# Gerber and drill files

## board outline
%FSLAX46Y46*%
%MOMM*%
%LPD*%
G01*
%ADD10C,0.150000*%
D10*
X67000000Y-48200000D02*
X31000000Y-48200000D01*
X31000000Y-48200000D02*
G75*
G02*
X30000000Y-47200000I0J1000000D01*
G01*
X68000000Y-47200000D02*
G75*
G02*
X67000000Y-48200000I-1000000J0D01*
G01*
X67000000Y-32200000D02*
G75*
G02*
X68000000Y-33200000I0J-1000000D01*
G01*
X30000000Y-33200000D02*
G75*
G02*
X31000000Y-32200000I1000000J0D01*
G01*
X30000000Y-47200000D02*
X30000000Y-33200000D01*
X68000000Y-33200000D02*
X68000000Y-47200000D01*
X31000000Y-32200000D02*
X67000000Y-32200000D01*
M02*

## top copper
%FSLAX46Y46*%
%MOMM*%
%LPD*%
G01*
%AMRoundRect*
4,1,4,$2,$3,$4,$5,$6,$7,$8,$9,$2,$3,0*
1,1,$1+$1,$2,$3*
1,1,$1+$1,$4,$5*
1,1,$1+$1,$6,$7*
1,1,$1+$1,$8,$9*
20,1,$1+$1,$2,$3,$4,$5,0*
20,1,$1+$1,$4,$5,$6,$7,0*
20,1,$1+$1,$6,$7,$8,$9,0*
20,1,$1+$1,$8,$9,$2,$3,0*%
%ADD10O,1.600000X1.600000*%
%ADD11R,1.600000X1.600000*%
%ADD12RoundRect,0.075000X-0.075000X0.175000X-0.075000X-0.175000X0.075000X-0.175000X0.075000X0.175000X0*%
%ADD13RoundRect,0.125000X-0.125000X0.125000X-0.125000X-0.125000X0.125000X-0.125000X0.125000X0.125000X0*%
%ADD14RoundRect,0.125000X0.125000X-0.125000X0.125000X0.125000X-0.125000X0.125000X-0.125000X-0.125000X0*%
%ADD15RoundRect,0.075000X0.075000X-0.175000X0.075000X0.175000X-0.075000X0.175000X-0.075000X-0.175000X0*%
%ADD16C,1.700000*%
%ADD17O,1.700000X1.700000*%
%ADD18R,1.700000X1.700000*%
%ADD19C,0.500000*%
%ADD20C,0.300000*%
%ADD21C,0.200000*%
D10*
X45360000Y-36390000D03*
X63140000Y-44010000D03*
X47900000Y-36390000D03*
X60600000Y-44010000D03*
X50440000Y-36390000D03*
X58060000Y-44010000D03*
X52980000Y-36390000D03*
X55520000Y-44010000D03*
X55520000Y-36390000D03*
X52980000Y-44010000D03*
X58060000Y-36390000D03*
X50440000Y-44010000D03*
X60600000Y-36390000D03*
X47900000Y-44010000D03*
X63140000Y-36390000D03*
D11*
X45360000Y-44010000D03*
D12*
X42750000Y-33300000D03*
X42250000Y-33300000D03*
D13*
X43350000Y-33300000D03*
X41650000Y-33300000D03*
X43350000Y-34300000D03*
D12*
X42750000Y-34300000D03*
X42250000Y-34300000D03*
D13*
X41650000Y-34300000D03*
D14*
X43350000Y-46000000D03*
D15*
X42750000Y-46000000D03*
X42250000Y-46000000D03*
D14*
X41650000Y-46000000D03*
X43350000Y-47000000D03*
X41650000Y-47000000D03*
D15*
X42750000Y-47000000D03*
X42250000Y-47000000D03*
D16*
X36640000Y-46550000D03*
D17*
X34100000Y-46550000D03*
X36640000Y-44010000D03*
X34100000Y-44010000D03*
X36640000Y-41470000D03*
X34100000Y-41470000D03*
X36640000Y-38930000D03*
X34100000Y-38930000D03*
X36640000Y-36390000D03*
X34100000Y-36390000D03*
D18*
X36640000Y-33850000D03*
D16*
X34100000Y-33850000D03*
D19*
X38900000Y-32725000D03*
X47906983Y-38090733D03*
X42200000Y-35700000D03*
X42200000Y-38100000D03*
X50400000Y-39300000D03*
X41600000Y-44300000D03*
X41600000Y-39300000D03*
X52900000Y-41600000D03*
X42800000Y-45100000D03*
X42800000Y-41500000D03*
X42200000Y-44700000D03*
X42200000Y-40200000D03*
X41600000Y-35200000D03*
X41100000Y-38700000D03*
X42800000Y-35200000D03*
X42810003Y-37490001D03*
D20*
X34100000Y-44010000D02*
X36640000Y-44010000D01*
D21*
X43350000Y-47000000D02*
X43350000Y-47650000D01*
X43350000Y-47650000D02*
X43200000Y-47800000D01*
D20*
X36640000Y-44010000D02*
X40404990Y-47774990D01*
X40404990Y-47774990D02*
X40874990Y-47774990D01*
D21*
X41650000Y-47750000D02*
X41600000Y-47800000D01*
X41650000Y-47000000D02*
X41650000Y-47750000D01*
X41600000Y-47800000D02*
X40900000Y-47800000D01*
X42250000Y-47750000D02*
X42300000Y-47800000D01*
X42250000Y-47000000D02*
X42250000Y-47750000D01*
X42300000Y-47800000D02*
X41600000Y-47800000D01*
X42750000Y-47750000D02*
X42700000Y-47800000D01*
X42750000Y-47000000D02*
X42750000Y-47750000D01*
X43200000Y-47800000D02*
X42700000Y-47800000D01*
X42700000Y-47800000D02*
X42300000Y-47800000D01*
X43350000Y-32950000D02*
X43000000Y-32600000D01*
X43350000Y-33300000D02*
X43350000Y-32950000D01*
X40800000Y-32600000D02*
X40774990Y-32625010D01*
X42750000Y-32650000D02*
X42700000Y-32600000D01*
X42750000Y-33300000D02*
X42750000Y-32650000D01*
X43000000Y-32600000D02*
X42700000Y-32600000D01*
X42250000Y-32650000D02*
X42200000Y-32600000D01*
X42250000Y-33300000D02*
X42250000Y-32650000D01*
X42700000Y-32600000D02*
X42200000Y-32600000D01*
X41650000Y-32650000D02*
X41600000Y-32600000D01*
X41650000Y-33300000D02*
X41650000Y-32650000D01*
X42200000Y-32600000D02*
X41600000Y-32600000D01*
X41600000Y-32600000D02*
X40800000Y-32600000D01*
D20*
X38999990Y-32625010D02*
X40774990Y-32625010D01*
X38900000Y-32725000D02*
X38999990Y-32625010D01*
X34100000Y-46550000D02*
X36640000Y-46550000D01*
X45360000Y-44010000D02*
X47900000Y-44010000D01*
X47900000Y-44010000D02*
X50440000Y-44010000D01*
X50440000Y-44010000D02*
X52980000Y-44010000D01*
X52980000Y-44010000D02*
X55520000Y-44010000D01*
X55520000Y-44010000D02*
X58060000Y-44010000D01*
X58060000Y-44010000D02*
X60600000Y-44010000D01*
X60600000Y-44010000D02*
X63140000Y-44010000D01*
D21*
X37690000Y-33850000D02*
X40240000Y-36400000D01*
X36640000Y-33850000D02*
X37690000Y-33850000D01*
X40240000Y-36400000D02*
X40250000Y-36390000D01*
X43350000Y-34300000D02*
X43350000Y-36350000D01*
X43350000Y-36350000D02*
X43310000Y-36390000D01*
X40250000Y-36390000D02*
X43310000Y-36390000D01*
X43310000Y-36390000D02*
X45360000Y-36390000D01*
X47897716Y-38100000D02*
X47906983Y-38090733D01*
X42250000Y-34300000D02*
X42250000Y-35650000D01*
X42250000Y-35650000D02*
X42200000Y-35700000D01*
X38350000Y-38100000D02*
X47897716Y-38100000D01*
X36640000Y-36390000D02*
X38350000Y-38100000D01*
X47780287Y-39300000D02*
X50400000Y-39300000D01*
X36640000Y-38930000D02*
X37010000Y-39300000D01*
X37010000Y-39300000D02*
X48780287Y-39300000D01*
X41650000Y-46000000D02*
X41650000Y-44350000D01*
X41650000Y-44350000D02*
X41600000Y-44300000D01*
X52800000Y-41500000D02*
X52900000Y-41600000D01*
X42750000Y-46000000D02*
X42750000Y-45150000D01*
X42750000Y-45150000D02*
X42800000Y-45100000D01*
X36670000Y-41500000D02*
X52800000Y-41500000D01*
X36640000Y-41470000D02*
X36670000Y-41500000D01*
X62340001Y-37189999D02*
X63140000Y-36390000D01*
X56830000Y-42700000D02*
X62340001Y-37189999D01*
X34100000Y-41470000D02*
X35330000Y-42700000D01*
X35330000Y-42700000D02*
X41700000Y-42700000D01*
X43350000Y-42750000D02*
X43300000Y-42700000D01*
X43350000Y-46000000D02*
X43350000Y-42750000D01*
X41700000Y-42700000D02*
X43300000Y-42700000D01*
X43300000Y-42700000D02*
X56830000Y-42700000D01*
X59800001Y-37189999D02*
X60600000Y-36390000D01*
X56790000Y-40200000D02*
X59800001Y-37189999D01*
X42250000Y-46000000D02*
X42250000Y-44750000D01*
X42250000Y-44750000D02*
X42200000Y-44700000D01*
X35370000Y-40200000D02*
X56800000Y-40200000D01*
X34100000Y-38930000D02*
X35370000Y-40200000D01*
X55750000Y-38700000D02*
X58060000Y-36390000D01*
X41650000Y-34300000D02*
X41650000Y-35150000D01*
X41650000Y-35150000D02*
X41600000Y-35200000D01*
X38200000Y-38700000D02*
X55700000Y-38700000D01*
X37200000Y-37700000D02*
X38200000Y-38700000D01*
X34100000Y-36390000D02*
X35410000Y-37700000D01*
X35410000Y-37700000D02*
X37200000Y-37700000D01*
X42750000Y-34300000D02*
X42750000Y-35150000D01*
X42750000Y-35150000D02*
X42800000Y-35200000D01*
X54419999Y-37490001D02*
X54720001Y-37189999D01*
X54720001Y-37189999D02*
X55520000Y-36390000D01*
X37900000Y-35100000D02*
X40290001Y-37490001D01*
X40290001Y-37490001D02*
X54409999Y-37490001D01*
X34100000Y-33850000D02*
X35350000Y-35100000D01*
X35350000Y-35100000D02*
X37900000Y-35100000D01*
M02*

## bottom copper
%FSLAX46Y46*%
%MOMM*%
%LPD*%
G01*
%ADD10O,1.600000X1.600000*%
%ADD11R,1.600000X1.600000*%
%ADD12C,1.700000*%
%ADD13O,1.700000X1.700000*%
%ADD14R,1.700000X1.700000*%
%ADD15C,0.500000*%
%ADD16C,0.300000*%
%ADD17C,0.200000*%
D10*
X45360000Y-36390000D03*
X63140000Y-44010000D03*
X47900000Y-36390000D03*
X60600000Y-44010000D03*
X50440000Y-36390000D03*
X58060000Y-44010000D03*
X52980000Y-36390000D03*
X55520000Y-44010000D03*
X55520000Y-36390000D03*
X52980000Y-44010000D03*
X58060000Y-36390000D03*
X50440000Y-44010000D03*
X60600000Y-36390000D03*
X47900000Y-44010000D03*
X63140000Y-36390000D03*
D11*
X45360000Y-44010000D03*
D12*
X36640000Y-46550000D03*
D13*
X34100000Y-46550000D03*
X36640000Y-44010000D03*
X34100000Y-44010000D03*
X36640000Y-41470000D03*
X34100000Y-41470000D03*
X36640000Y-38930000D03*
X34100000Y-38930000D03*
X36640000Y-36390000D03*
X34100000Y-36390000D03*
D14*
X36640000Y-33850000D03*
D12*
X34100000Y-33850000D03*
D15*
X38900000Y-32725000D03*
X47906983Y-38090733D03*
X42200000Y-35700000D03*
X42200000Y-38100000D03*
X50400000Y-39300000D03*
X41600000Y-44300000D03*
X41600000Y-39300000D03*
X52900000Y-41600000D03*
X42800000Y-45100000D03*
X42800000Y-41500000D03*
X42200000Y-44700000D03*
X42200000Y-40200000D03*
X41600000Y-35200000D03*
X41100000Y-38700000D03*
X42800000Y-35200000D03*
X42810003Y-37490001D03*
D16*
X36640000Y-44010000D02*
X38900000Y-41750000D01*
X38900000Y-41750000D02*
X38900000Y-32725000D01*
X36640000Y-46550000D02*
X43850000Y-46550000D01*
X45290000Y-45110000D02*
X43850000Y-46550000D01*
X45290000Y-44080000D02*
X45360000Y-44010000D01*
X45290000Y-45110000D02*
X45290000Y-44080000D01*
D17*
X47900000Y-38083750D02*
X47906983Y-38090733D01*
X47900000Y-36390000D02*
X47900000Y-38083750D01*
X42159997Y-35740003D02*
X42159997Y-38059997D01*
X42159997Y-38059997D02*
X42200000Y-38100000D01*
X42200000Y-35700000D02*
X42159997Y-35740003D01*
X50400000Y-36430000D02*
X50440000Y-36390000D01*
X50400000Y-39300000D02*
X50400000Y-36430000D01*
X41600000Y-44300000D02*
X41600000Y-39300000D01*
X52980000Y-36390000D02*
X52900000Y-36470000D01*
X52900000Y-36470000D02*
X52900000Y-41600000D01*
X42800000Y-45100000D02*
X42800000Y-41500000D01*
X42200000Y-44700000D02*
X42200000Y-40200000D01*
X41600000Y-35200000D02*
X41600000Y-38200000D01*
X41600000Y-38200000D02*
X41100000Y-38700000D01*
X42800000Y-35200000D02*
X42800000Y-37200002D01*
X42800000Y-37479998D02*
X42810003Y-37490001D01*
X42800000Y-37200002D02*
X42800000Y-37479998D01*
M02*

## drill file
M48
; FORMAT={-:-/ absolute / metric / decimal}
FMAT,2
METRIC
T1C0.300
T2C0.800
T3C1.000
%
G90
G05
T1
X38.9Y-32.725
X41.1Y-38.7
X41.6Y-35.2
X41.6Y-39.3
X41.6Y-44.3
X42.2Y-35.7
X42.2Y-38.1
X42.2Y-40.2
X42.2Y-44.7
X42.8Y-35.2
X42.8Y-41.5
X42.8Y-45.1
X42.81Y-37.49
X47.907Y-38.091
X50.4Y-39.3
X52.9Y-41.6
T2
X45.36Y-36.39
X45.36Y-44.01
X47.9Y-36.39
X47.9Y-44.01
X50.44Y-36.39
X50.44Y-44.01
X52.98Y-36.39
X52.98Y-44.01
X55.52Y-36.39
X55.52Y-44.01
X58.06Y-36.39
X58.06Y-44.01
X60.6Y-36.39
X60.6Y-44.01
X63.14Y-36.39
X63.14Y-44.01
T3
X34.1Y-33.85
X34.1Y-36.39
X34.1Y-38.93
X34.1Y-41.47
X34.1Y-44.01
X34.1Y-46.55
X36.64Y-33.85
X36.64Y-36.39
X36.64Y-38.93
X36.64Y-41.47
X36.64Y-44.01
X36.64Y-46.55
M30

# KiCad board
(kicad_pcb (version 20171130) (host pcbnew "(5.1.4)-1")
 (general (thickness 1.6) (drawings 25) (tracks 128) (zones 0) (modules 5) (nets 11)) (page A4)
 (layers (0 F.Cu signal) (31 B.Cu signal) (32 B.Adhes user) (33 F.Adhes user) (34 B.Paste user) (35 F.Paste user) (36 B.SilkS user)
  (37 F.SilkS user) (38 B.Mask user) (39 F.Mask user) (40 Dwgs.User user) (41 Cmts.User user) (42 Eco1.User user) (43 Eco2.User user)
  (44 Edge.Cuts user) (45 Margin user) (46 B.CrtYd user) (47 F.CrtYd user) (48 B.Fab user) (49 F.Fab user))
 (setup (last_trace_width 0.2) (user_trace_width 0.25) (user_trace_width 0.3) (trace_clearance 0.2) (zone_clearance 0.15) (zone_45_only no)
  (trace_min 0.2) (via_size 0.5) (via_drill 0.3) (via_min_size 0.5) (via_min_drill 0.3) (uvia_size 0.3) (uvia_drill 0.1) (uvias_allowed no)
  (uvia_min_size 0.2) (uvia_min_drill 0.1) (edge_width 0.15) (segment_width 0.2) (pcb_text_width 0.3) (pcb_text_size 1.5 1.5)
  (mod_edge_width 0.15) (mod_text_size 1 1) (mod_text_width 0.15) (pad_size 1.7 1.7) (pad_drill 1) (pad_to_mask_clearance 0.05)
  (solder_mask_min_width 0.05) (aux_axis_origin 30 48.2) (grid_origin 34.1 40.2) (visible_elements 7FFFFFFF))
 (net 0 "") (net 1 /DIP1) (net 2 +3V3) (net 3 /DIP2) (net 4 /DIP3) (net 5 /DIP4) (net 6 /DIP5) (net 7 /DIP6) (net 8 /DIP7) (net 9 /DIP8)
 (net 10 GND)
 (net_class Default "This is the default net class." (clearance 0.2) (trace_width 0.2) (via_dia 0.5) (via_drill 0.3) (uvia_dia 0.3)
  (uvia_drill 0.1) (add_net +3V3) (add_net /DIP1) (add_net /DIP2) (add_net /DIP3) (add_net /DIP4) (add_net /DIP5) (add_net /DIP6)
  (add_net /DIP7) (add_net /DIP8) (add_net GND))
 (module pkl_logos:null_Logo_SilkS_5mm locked (layer B.Cu) (at 55.52 40.2 90)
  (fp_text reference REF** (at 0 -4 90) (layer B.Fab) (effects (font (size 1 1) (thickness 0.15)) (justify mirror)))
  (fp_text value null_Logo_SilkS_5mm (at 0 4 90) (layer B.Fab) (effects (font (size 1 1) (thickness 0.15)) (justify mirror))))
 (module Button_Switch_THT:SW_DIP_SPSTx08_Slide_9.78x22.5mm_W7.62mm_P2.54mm (layer F.Cu) (at 45.36 44.01 90)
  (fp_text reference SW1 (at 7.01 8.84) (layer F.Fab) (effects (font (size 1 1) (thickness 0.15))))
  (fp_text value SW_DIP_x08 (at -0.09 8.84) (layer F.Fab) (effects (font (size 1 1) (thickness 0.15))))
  (pad 16 thru_hole oval (at 7.62 0 90) (size 1.6 1.6) (drill 0.8) (layers *.Cu *.Mask) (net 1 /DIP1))
  (pad 8 thru_hole oval (at 0 17.78 90) (size 1.6 1.6) (drill 0.8) (layers *.Cu *.Mask) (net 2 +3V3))
  (pad 15 thru_hole oval (at 7.62 2.54 90) (size 1.6 1.6) (drill 0.8) (layers *.Cu *.Mask) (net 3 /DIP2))
  (pad 7 thru_hole oval (at 0 15.24 90) (size 1.6 1.6) (drill 0.8) (layers *.Cu *.Mask) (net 2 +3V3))
  (pad 14 thru_hole oval (at 7.62 5.08 90) (size 1.6 1.6) (drill 0.8) (layers *.Cu *.Mask) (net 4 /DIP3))
  (pad 6 thru_hole oval (at 0 12.7 90) (size 1.6 1.6) (drill 0.8) (layers *.Cu *.Mask) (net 2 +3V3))
  (pad 13 thru_hole oval (at 7.62 7.62 90) (size 1.6 1.6) (drill 0.8) (layers *.Cu *.Mask) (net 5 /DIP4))
  (pad 5 thru_hole oval (at 0 10.16 90) (size 1.6 1.6) (drill 0.8) (layers *.Cu *.Mask) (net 2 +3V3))
  (pad 12 thru_hole oval (at 7.62 10.16 90) (size 1.6 1.6) (drill 0.8) (layers *.Cu *.Mask) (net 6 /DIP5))
  (pad 4 thru_hole oval (at 0 7.62 90) (size 1.6 1.6) (drill 0.8) (layers *.Cu *.Mask) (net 2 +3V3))
  (pad 11 thru_hole oval (at 7.62 12.7 90) (size 1.6 1.6) (drill 0.8) (layers *.Cu *.Mask) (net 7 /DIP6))
  (pad 3 thru_hole oval (at 0 5.08 90) (size 1.6 1.6) (drill 0.8) (layers *.Cu *.Mask) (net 2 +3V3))
  (pad 10 thru_hole oval (at 7.62 15.24 90) (size 1.6 1.6) (drill 0.8) (layers *.Cu *.Mask) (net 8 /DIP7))
  (pad 2 thru_hole oval (at 0 2.54 90) (size 1.6 1.6) (drill 0.8) (layers *.Cu *.Mask) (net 2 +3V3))
  (pad 9 thru_hole oval (at 7.62 17.78 90) (size 1.6 1.6) (drill 0.8) (layers *.Cu *.Mask) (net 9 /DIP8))
  (pad 1 thru_hole rect (at 0 0 90) (size 1.6 1.6) (drill 0.8) (layers *.Cu *.Mask) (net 2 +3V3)))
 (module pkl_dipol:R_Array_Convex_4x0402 (layer F.Cu) (at 42.5 33.8 270) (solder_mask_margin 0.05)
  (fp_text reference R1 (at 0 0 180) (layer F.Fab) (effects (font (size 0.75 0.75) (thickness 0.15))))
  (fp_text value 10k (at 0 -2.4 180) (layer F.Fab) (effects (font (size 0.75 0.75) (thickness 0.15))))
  (pad 3 smd roundrect (at -0.5 -0.25 270) (size 0.5 0.3) (layers F.Cu F.Paste F.Mask) (roundrect_rratio 0.25) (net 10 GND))
  (pad 5 smd roundrect (at -0.5 0.25 270) (size 0.5 0.3) (layers F.Cu F.Paste F.Mask) (roundrect_rratio 0.25) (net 10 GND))
  (pad 1 smd roundrect (at -0.5 -0.85 270) (size 0.5 0.5) (layers F.Cu F.Paste F.Mask) (roundrect_rratio 0.25) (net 10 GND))
  (pad 7 smd roundrect (at -0.5 0.85 270) (size 0.5 0.5) (layers F.Cu F.Paste F.Mask) (roundrect_rratio 0.25) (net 10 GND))
  (pad 2 smd roundrect (at 0.5 -0.85 270) (size 0.5 0.5) (layers F.Cu F.Paste F.Mask) (roundrect_rratio 0.25) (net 1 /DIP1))
  (pad 4 smd roundrect (at 0.5 -0.25 270) (size 0.5 0.3) (layers F.Cu F.Paste F.Mask) (roundrect_rratio 0.25) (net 6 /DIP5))
  (pad 6 smd roundrect (at 0.5 0.25 270) (size 0.5 0.3) (layers F.Cu F.Paste F.Mask) (roundrect_rratio 0.25) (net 3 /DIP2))
  (pad 8 smd roundrect (at 0.5 0.85 270) (size 0.5 0.5) (layers F.Cu F.Paste F.Mask) (roundrect_rratio 0.25) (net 7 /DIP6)))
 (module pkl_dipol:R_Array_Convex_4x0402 (layer F.Cu) (at 42.5 46.5 90) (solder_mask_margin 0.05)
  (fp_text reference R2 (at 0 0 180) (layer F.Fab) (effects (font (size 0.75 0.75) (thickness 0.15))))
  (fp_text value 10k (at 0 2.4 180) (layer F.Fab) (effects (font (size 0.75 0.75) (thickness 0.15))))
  (pad 8 smd roundrect (at 0.5 0.85 90) (size 0.5 0.5) (layers F.Cu F.Paste F.Mask) (roundrect_rratio 0.25) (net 9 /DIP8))
  (pad 6 smd roundrect (at 0.5 0.25 90) (size 0.5 0.3) (layers F.Cu F.Paste F.Mask) (roundrect_rratio 0.25) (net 5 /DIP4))
  (pad 4 smd roundrect (at 0.5 -0.25 90) (size 0.5 0.3) (layers F.Cu F.Paste F.Mask) (roundrect_rratio 0.25) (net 8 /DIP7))
  (pad 2 smd roundrect (at 0.5 -0.85 90) (size 0.5 0.5) (layers F.Cu F.Paste F.Mask) (roundrect_rratio 0.25) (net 4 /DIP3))
  (pad 7 smd roundrect (at -0.5 0.85 90) (size 0.5 0.5) (layers F.Cu F.Paste F.Mask) (roundrect_rratio 0.25) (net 10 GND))
  (pad 1 smd roundrect (at -0.5 -0.85 90) (size 0.5 0.5) (layers F.Cu F.Paste F.Mask) (roundrect_rratio 0.25) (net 10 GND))
  (pad 5 smd roundrect (at -0.5 0.25 90) (size 0.5 0.3) (layers F.Cu F.Paste F.Mask) (roundrect_rratio 0.25) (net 10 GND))
  (pad 3 smd roundrect (at -0.5 -0.25 90) (size 0.5 0.3) (layers F.Cu F.Paste F.Mask) (roundrect_rratio 0.25) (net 10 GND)))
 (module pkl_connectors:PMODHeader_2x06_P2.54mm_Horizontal (layer F.Cu) (at 36.64 46.55 180)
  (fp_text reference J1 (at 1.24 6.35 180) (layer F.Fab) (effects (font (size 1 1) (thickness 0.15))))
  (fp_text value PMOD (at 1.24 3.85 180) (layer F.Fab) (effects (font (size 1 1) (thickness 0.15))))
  (pad 6 thru_hole circle (at 0 0 180) (size 1.7 1.7) (drill 1) (layers *.Cu *.Mask) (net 2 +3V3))
  (pad 12 thru_hole oval (at 2.54 0 180) (size 1.7 1.7) (drill 1) (layers *.Cu *.Mask) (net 2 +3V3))
  (pad 5 thru_hole oval (at 0 2.54 180) (size 1.7 1.7) (drill 1) (layers *.Cu *.Mask) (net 10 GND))
  (pad 11 thru_hole oval (at 2.54 2.54 180) (size 1.7 1.7) (drill 1) (layers *.Cu *.Mask) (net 10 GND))
  (pad 4 thru_hole oval (at 0 5.08 180) (size 1.7 1.7) (drill 1) (layers *.Cu *.Mask) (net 5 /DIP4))
  (pad 10 thru_hole oval (at 2.54 5.08 180) (size 1.7 1.7) (drill 1) (layers *.Cu *.Mask) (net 9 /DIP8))
  (pad 3 thru_hole oval (at 0 7.62 180) (size 1.7 1.7) (drill 1) (layers *.Cu *.Mask) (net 4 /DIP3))
  (pad 9 thru_hole oval (at 2.54 7.62 180) (size 1.7 1.7) (drill 1) (layers *.Cu *.Mask) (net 8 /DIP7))
  (pad 2 thru_hole oval (at 0 10.16 180) (size 1.7 1.7) (drill 1) (layers *.Cu *.Mask) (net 3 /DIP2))
  (pad 8 thru_hole oval (at 2.54 10.16 180) (size 1.7 1.7) (drill 1) (layers *.Cu *.Mask) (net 7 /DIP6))
  (pad 1 thru_hole rect (at 0 12.7 180) (size 1.7 1.7) (drill 1) (layers *.Cu *.Mask) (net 1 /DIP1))
  (pad 7 thru_hole circle (at 2.54 12.7 180) (size 1.7 1.7) (drill 1) (layers *.Cu *.Mask) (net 6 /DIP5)))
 (gr_line (start 67 48.2) (end 31 48.2) (layer Edge.Cuts) (width 0.15))
 (gr_arc (start 31 47.2) (end 30 47.2) (angle -90) (layer Edge.Cuts) (width 0.15))
 (gr_arc (start 67 47.2) (end 67 48.2) (angle -90) (layer Edge.Cuts) (width 0.15))
 (gr_arc (start 67 33.2) (end 68 33.2) (angle -90) (layer Edge.Cuts) (width 0.15))
 (gr_arc (start 31 33.2) (end 31 32.2) (angle -90) (layer Edge.Cuts) (width 0.15))
 (gr_line (start 30 47.2) (end 30 33.2) (layer Edge.Cuts) (width 0.15))
 (gr_line (start 68 33.2) (end 68 47.2) (layer Edge.Cuts) (width 0.15))
 (gr_line (start 31 32.2) (end 67 32.2) (layer Edge.Cuts) (width 0.15))
 (segment (start 34.1 44.01) (end 36.64 44.01) (width 0.3) (layer F.Cu) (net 10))
 (segment (start 43.35 47) (end 43.35 47.65) (width 0.2) (layer F.Cu) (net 10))
 (segment (start 43.35 47.65) (end 43.2 47.8) (width 0.2) (layer F.Cu) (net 10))
 (segment (start 36.64 44.01) (end 40.40499 47.77499) (width 0.3) (layer F.Cu) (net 10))
 (segment (start 40.40499 47.77499) (end 40.87499 47.77499) (width 0.3) (layer F.Cu) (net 10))
 (segment (start 41.65 47.75) (end 41.6 47.8) (width 0.2) (layer F.Cu) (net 10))
 (segment (start 41.65 47) (end 41.65 47.75) (width 0.2) (layer F.Cu) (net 10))
 (segment (start 41.6 47.8) (end 40.9 47.8) (width 0.2) (layer F.Cu) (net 10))
 (segment (start 42.25 47.75) (end 42.3 47.8) (width 0.2) (layer F.Cu) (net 10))
 (segment (start 42.25 47) (end 42.25 47.75) (width 0.2) (layer F.Cu) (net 10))
 (segment (start 42.3 47.8) (end 41.6 47.8) (width 0.2) (layer F.Cu) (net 10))
 (segment (start 42.75 47.75) (end 42.7 47.8) (width 0.2) (layer F.Cu) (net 10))
 (segment (start 42.75 47) (end 42.75 47.75) (width 0.2) (layer F.Cu) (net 10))
 (segment (start 43.2 47.8) (end 42.7 47.8) (width 0.2) (layer F.Cu) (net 10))
 (segment (start 42.7 47.8) (end 42.3 47.8) (width 0.2) (layer F.Cu) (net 10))
 (via (at 38.9 32.725) (size 0.5) (drill 0.3) (layers F.Cu B.Cu) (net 10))
 (segment (start 36.64 44.01) (end 38.9 41.75) (width 0.3) (layer B.Cu) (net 10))
 (segment (start 38.9 41.75) (end 38.9 32.725) (width 0.3) (layer B.Cu) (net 10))
 (segment (start 43.35 32.95) (end 43 32.6) (width 0.2) (layer F.Cu) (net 10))
 (segment (start 43.35 33.3) (end 43.35 32.95) (width 0.2) (layer F.Cu) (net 10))
 (segment (start 40.8 32.6) (end 40.77499 32.62501) (width 0.2) (layer F.Cu) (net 10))
 (segment (start 42.75 32.65) (end 42.7 32.6) (width 0.2) (layer F.Cu) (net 10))
 (segment (start 42.75 33.3) (end 42.75 32.65) (width 0.2) (layer F.Cu) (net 10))
 (segment (start 43 32.6) (end 42.7 32.6) (width 0.2) (layer F.Cu) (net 10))
 (segment (start 42.25 32.65) (end 42.2 32.6) (width 0.2) (layer F.Cu) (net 10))
 (segment (start 42.25 33.3) (end 42.25 32.65) (width 0.2) (layer F.Cu) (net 10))
 (segment (start 42.7 32.6) (end 42.2 32.6) (width 0.2) (layer F.Cu) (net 10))
 (segment (start 41.65 32.65) (end 41.6 32.6) (width 0.2) (layer F.Cu) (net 10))
 (segment (start 41.65 33.3) (end 41.65 32.65) (width 0.2) (layer F.Cu) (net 10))
 (segment (start 42.2 32.6) (end 41.6 32.6) (width 0.2) (layer F.Cu) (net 10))
 (segment (start 41.6 32.6) (end 40.8 32.6) (width 0.2) (layer F.Cu) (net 10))
 (segment (start 38.99999 32.62501) (end 40.77499 32.62501) (width 0.3) (layer F.Cu) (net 10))
 (segment (start 38.9 32.725) (end 38.99999 32.62501) (width 0.3) (layer F.Cu) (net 10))
 (segment (start 34.1 46.55) (end 36.64 46.55) (width 0.3) (layer F.Cu) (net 2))
 (segment (start 45.36 44.01) (end 47.9 44.01) (width 0.3) (layer F.Cu) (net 2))
 (segment (start 47.9 44.01) (end 50.44 44.01) (width 0.3) (layer F.Cu) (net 2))
 (segment (start 50.44 44.01) (end 52.98 44.01) (width 0.3) (layer F.Cu) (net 2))
 (segment (start 52.98 44.01) (end 55.52 44.01) (width 0.3) (layer F.Cu) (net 2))
 (segment (start 55.52 44.01) (end 58.06 44.01) (width 0.3) (layer F.Cu) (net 2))
 (segment (start 58.06 44.01) (end 60.6 44.01) (width 0.3) (layer F.Cu) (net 2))
 (segment (start 60.6 44.01) (end 63.14 44.01) (width 0.3) (layer F.Cu) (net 2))
 (segment (start 36.64 46.55) (end 43.85 46.55) (width 0.3) (layer B.Cu) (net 2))
 (segment (start 45.29 45.11) (end 43.85 46.55) (width 0.3) (layer B.Cu) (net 2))
 (segment (start 45.29 44.08) (end 45.36 44.01) (width 0.3) (layer B.Cu) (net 2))
 (segment (start 45.29 45.11) (end 45.29 44.08) (width 0.3) (layer B.Cu) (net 2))
 (segment (start 37.69 33.85) (end 40.24 36.4) (width 0.2) (layer F.Cu) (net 1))
 (segment (start 36.64 33.85) (end 37.69 33.85) (width 0.2) (layer F.Cu) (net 1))
 (segment (start 40.24 36.4) (end 40.25 36.39) (width 0.2) (layer F.Cu) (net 1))
 (segment (start 43.35 34.3) (end 43.35 36.35) (width 0.2) (layer F.Cu) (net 1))
 (segment (start 43.35 36.35) (end 43.31 36.39) (width 0.2) (layer F.Cu) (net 1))
 (segment (start 40.25 36.39) (end 43.31 36.39) (width 0.2) (layer F.Cu) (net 1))
 (segment (start 43.31 36.39) (end 45.36 36.39) (width 0.2) (layer F.Cu) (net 1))
 (via (at 47.906983 38.090733) (size 0.5) (drill 0.3) (layers F.Cu B.Cu) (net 3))
 (segment (start 47.9 38.08375) (end 47.906983 38.090733) (width 0.2) (layer B.Cu) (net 3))
 (segment (start 47.9 36.39) (end 47.9 38.08375) (width 0.2) (layer B.Cu) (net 3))
 (segment (start 47.897716 38.1) (end 47.906983 38.090733) (width 0.2) (layer F.Cu) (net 3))
 (via (at 42.2 35.7) (size 0.5) (drill 0.3) (layers F.Cu B.Cu) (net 3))
 (segment (start 42.25 34.3) (end 42.25 35.65) (width 0.2) (layer F.Cu) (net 3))
 (segment (start 42.25 35.65) (end 42.2 35.7) (width 0.2) (layer F.Cu) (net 3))
 (via (at 42.2 38.1) (size 0.5) (drill 0.3) (layers F.Cu B.Cu) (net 3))
 (segment (start 42.159997 35.740003) (end 42.159997 38.059997) (width 0.2) (layer B.Cu) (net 3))
 (segment (start 42.159997 38.059997) (end 42.2 38.1) (width 0.2) (layer B.Cu) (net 3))
 (segment (start 42.2 35.7) (end 42.159997 35.740003) (width 0.2) (layer B.Cu) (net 3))
 (segment (start 38.35 38.1) (end 47.897716 38.1) (width 0.2) (layer F.Cu) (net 3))
 (segment (start 36.64 36.39) (end 38.35 38.1) (width 0.2) (layer F.Cu) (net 3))
 (via (at 50.4 39.3) (size 0.5) (drill 0.3) (layers F.Cu B.Cu) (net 4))
 (segment (start 50.4 36.43) (end 50.44 36.39) (width 0.2) (layer B.Cu) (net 4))
 (segment (start 50.4 39.3) (end 50.4 36.43) (width 0.2) (layer B.Cu) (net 4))
 (segment (start 47.780287 39.3) (end 50.4 39.3) (width 0.2) (layer F.Cu) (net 4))
 (segment (start 36.64 38.93) (end 37.01 39.3) (width 0.2) (layer F.Cu) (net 4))
 (segment (start 37.01 39.3) (end 48.780287 39.3) (width 0.2) (layer F.Cu) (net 4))
 (via (at 41.6 44.3) (size 0.5) (drill 0.3) (layers F.Cu B.Cu) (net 4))
 (segment (start 41.65 46) (end 41.65 44.35) (width 0.2) (layer F.Cu) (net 4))
 (segment (start 41.65 44.35) (end 41.6 44.3) (width 0.2) (layer F.Cu) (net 4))
 (via (at 41.6 39.3) (size 0.5) (drill 0.3) (layers F.Cu B.Cu) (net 4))
 (segment (start 41.6 44.3) (end 41.6 39.3) (width 0.2) (layer B.Cu) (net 4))
 (segment (start 52.8 41.5) (end 52.9 41.6) (width 0.2) (layer F.Cu) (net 5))
 (via (at 52.9 41.6) (size 0.5) (drill 0.3) (layers F.Cu B.Cu) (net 5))
 (segment (start 52.98 36.39) (end 52.9 36.47) (width 0.2) (layer B.Cu) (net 5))
 (segment (start 52.9 36.47) (end 52.9 41.6) (width 0.2) (layer B.Cu) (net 5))
 (via (at 42.8 45.1) (size 0.5) (drill 0.3) (layers F.Cu B.Cu) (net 5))
 (segment (start 42.75 46) (end 42.75 45.15) (width 0.2) (layer F.Cu) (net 5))
 (segment (start 42.75 45.15) (end 42.8 45.1) (width 0.2) (layer F.Cu) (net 5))
 (via (at 42.8 41.5) (size 0.5) (drill 0.3) (layers F.Cu B.Cu) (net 5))
 (segment (start 42.8 45.1) (end 42.8 41.5) (width 0.2) (layer B.Cu) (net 5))
 (segment (start 36.67 41.5) (end 52.8 41.5) (width 0.2) (layer F.Cu) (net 5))
 (segment (start 36.64 41.47) (end 36.67 41.5) (width 0.2) (layer F.Cu) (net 5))
 (segment (start 62.340001 37.189999) (end 63.14 36.39) (width 0.2) (layer F.Cu) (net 9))
 (segment (start 56.83 42.7) (end 62.340001 37.189999) (width 0.2) (layer F.Cu) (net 9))
 (segment (start 34.1 41.47) (end 35.33 42.7) (width 0.2) (layer F.Cu) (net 9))
 (segment (start 35.33 42.7) (end 41.7 42.7) (width 0.2) (layer F.Cu) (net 9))
 (segment (start 43.35 42.75) (end 43.3 42.7) (width 0.2) (layer F.Cu) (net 9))
 (segment (start 43.35 46) (end 43.35 42.75) (width 0.2) (layer F.Cu) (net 9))
 (segment (start 41.7 42.7) (end 43.3 42.7) (width 0.2) (layer F.Cu) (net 9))
 (segment (start 43.3 42.7) (end 56.83 42.7) (width 0.2) (layer F.Cu) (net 9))
 (segment (start 59.800001 37.189999) (end 60.6 36.39) (width 0.2) (layer F.Cu) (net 8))
 (segment (start 56.79 40.2) (end 59.800001 37.189999) (width 0.2) (layer F.Cu) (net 8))
 (via (at 42.2 44.7) (size 0.5) (drill 0.3) (layers F.Cu B.Cu) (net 8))
 (segment (start 42.25 46) (end 42.25 44.75) (width 0.2) (layer F.Cu) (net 8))
 (segment (start 42.25 44.75) (end 42.2 44.7) (width 0.2) (layer F.Cu) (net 8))
 (via (at 42.2 40.2) (size 0.5) (drill 0.3) (layers F.Cu B.Cu) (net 8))
 (segment (start 42.2 44.7) (end 42.2 40.2) (width 0.2) (layer B.Cu) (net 8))
 (segment (start 35.37 40.2) (end 56.8 40.2) (width 0.2) (layer F.Cu) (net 8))
 (segment (start 34.1 38.93) (end 35.37 40.2) (width 0.2) (layer F.Cu) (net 8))
 (segment (start 55.75 38.7) (end 58.06 36.39) (width 0.2) (layer F.Cu) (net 7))
 (via (at 41.6 35.2) (size 0.5) (drill 0.3) (layers F.Cu B.Cu) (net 7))
 (segment (start 41.65 34.3) (end 41.65 35.15) (width 0.2) (layer F.Cu) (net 7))
 (segment (start 41.65 35.15) (end 41.6 35.2) (width 0.2) (layer F.Cu) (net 7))
 (segment (start 41.6 35.2) (end 41.6 38.2) (width 0.2) (layer B.Cu) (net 7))
 (via (at 41.1 38.7) (size 0.5) (drill 0.3) (layers F.Cu B.Cu) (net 7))
 (segment (start 41.6 38.2) (end 41.1 38.7) (width 0.2) (layer B.Cu) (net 7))
 (segment (start 38.2 38.7) (end 55.7 38.7) (width 0.2) (layer F.Cu) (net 7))
 (segment (start 37.2 37.7) (end 38.2 38.7) (width 0.2) (layer F.Cu) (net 7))
 (segment (start 34.1 36.39) (end 35.41 37.7) (width 0.2) (layer F.Cu) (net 7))
 (segment (start 35.41 37.7) (end 37.2 37.7) (width 0.2) (layer F.Cu) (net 7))
 (via (at 42.8 35.2) (size 0.5) (drill 0.3) (layers F.Cu B.Cu) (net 6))
 (segment (start 42.75 34.3) (end 42.75 35.15) (width 0.2) (layer F.Cu) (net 6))
 (segment (start 42.75 35.15) (end 42.8 35.2) (width 0.2) (layer F.Cu) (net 6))
 (segment (start 42.8 35.2) (end 42.8 37.200002) (width 0.2) (layer B.Cu) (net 6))
 (via (at 42.810003 37.490001) (size 0.5) (drill 0.3) (layers F.Cu B.Cu) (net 6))
 (segment (start 42.8 37.479998) (end 42.810003 37.490001) (width 0.2) (layer B.Cu) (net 6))
 (segment (start 42.8 37.200002) (end 42.8 37.479998) (width 0.2) (layer B.Cu) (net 6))
 (segment (start 54.419999 37.490001) (end 54.720001 37.189999) (width 0.2) (layer F.Cu) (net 6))
 (segment (start 54.720001 37.189999) (end 55.52 36.39) (width 0.2) (layer F.Cu) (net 6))
 (segment (start 37.9 35.1) (end 40.290001 37.490001) (width 0.2) (layer F.Cu) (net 6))
 (segment (start 40.290001 37.490001) (end 54.409999 37.490001) (width 0.2) (layer F.Cu) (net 6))
 (segment (start 34.1 33.85) (end 35.35 35.1) (width 0.2) (layer F.Cu) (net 6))
 (segment (start 35.35 35.1) (end 37.9 35.1) (width 0.2) (layer F.Cu) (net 6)))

